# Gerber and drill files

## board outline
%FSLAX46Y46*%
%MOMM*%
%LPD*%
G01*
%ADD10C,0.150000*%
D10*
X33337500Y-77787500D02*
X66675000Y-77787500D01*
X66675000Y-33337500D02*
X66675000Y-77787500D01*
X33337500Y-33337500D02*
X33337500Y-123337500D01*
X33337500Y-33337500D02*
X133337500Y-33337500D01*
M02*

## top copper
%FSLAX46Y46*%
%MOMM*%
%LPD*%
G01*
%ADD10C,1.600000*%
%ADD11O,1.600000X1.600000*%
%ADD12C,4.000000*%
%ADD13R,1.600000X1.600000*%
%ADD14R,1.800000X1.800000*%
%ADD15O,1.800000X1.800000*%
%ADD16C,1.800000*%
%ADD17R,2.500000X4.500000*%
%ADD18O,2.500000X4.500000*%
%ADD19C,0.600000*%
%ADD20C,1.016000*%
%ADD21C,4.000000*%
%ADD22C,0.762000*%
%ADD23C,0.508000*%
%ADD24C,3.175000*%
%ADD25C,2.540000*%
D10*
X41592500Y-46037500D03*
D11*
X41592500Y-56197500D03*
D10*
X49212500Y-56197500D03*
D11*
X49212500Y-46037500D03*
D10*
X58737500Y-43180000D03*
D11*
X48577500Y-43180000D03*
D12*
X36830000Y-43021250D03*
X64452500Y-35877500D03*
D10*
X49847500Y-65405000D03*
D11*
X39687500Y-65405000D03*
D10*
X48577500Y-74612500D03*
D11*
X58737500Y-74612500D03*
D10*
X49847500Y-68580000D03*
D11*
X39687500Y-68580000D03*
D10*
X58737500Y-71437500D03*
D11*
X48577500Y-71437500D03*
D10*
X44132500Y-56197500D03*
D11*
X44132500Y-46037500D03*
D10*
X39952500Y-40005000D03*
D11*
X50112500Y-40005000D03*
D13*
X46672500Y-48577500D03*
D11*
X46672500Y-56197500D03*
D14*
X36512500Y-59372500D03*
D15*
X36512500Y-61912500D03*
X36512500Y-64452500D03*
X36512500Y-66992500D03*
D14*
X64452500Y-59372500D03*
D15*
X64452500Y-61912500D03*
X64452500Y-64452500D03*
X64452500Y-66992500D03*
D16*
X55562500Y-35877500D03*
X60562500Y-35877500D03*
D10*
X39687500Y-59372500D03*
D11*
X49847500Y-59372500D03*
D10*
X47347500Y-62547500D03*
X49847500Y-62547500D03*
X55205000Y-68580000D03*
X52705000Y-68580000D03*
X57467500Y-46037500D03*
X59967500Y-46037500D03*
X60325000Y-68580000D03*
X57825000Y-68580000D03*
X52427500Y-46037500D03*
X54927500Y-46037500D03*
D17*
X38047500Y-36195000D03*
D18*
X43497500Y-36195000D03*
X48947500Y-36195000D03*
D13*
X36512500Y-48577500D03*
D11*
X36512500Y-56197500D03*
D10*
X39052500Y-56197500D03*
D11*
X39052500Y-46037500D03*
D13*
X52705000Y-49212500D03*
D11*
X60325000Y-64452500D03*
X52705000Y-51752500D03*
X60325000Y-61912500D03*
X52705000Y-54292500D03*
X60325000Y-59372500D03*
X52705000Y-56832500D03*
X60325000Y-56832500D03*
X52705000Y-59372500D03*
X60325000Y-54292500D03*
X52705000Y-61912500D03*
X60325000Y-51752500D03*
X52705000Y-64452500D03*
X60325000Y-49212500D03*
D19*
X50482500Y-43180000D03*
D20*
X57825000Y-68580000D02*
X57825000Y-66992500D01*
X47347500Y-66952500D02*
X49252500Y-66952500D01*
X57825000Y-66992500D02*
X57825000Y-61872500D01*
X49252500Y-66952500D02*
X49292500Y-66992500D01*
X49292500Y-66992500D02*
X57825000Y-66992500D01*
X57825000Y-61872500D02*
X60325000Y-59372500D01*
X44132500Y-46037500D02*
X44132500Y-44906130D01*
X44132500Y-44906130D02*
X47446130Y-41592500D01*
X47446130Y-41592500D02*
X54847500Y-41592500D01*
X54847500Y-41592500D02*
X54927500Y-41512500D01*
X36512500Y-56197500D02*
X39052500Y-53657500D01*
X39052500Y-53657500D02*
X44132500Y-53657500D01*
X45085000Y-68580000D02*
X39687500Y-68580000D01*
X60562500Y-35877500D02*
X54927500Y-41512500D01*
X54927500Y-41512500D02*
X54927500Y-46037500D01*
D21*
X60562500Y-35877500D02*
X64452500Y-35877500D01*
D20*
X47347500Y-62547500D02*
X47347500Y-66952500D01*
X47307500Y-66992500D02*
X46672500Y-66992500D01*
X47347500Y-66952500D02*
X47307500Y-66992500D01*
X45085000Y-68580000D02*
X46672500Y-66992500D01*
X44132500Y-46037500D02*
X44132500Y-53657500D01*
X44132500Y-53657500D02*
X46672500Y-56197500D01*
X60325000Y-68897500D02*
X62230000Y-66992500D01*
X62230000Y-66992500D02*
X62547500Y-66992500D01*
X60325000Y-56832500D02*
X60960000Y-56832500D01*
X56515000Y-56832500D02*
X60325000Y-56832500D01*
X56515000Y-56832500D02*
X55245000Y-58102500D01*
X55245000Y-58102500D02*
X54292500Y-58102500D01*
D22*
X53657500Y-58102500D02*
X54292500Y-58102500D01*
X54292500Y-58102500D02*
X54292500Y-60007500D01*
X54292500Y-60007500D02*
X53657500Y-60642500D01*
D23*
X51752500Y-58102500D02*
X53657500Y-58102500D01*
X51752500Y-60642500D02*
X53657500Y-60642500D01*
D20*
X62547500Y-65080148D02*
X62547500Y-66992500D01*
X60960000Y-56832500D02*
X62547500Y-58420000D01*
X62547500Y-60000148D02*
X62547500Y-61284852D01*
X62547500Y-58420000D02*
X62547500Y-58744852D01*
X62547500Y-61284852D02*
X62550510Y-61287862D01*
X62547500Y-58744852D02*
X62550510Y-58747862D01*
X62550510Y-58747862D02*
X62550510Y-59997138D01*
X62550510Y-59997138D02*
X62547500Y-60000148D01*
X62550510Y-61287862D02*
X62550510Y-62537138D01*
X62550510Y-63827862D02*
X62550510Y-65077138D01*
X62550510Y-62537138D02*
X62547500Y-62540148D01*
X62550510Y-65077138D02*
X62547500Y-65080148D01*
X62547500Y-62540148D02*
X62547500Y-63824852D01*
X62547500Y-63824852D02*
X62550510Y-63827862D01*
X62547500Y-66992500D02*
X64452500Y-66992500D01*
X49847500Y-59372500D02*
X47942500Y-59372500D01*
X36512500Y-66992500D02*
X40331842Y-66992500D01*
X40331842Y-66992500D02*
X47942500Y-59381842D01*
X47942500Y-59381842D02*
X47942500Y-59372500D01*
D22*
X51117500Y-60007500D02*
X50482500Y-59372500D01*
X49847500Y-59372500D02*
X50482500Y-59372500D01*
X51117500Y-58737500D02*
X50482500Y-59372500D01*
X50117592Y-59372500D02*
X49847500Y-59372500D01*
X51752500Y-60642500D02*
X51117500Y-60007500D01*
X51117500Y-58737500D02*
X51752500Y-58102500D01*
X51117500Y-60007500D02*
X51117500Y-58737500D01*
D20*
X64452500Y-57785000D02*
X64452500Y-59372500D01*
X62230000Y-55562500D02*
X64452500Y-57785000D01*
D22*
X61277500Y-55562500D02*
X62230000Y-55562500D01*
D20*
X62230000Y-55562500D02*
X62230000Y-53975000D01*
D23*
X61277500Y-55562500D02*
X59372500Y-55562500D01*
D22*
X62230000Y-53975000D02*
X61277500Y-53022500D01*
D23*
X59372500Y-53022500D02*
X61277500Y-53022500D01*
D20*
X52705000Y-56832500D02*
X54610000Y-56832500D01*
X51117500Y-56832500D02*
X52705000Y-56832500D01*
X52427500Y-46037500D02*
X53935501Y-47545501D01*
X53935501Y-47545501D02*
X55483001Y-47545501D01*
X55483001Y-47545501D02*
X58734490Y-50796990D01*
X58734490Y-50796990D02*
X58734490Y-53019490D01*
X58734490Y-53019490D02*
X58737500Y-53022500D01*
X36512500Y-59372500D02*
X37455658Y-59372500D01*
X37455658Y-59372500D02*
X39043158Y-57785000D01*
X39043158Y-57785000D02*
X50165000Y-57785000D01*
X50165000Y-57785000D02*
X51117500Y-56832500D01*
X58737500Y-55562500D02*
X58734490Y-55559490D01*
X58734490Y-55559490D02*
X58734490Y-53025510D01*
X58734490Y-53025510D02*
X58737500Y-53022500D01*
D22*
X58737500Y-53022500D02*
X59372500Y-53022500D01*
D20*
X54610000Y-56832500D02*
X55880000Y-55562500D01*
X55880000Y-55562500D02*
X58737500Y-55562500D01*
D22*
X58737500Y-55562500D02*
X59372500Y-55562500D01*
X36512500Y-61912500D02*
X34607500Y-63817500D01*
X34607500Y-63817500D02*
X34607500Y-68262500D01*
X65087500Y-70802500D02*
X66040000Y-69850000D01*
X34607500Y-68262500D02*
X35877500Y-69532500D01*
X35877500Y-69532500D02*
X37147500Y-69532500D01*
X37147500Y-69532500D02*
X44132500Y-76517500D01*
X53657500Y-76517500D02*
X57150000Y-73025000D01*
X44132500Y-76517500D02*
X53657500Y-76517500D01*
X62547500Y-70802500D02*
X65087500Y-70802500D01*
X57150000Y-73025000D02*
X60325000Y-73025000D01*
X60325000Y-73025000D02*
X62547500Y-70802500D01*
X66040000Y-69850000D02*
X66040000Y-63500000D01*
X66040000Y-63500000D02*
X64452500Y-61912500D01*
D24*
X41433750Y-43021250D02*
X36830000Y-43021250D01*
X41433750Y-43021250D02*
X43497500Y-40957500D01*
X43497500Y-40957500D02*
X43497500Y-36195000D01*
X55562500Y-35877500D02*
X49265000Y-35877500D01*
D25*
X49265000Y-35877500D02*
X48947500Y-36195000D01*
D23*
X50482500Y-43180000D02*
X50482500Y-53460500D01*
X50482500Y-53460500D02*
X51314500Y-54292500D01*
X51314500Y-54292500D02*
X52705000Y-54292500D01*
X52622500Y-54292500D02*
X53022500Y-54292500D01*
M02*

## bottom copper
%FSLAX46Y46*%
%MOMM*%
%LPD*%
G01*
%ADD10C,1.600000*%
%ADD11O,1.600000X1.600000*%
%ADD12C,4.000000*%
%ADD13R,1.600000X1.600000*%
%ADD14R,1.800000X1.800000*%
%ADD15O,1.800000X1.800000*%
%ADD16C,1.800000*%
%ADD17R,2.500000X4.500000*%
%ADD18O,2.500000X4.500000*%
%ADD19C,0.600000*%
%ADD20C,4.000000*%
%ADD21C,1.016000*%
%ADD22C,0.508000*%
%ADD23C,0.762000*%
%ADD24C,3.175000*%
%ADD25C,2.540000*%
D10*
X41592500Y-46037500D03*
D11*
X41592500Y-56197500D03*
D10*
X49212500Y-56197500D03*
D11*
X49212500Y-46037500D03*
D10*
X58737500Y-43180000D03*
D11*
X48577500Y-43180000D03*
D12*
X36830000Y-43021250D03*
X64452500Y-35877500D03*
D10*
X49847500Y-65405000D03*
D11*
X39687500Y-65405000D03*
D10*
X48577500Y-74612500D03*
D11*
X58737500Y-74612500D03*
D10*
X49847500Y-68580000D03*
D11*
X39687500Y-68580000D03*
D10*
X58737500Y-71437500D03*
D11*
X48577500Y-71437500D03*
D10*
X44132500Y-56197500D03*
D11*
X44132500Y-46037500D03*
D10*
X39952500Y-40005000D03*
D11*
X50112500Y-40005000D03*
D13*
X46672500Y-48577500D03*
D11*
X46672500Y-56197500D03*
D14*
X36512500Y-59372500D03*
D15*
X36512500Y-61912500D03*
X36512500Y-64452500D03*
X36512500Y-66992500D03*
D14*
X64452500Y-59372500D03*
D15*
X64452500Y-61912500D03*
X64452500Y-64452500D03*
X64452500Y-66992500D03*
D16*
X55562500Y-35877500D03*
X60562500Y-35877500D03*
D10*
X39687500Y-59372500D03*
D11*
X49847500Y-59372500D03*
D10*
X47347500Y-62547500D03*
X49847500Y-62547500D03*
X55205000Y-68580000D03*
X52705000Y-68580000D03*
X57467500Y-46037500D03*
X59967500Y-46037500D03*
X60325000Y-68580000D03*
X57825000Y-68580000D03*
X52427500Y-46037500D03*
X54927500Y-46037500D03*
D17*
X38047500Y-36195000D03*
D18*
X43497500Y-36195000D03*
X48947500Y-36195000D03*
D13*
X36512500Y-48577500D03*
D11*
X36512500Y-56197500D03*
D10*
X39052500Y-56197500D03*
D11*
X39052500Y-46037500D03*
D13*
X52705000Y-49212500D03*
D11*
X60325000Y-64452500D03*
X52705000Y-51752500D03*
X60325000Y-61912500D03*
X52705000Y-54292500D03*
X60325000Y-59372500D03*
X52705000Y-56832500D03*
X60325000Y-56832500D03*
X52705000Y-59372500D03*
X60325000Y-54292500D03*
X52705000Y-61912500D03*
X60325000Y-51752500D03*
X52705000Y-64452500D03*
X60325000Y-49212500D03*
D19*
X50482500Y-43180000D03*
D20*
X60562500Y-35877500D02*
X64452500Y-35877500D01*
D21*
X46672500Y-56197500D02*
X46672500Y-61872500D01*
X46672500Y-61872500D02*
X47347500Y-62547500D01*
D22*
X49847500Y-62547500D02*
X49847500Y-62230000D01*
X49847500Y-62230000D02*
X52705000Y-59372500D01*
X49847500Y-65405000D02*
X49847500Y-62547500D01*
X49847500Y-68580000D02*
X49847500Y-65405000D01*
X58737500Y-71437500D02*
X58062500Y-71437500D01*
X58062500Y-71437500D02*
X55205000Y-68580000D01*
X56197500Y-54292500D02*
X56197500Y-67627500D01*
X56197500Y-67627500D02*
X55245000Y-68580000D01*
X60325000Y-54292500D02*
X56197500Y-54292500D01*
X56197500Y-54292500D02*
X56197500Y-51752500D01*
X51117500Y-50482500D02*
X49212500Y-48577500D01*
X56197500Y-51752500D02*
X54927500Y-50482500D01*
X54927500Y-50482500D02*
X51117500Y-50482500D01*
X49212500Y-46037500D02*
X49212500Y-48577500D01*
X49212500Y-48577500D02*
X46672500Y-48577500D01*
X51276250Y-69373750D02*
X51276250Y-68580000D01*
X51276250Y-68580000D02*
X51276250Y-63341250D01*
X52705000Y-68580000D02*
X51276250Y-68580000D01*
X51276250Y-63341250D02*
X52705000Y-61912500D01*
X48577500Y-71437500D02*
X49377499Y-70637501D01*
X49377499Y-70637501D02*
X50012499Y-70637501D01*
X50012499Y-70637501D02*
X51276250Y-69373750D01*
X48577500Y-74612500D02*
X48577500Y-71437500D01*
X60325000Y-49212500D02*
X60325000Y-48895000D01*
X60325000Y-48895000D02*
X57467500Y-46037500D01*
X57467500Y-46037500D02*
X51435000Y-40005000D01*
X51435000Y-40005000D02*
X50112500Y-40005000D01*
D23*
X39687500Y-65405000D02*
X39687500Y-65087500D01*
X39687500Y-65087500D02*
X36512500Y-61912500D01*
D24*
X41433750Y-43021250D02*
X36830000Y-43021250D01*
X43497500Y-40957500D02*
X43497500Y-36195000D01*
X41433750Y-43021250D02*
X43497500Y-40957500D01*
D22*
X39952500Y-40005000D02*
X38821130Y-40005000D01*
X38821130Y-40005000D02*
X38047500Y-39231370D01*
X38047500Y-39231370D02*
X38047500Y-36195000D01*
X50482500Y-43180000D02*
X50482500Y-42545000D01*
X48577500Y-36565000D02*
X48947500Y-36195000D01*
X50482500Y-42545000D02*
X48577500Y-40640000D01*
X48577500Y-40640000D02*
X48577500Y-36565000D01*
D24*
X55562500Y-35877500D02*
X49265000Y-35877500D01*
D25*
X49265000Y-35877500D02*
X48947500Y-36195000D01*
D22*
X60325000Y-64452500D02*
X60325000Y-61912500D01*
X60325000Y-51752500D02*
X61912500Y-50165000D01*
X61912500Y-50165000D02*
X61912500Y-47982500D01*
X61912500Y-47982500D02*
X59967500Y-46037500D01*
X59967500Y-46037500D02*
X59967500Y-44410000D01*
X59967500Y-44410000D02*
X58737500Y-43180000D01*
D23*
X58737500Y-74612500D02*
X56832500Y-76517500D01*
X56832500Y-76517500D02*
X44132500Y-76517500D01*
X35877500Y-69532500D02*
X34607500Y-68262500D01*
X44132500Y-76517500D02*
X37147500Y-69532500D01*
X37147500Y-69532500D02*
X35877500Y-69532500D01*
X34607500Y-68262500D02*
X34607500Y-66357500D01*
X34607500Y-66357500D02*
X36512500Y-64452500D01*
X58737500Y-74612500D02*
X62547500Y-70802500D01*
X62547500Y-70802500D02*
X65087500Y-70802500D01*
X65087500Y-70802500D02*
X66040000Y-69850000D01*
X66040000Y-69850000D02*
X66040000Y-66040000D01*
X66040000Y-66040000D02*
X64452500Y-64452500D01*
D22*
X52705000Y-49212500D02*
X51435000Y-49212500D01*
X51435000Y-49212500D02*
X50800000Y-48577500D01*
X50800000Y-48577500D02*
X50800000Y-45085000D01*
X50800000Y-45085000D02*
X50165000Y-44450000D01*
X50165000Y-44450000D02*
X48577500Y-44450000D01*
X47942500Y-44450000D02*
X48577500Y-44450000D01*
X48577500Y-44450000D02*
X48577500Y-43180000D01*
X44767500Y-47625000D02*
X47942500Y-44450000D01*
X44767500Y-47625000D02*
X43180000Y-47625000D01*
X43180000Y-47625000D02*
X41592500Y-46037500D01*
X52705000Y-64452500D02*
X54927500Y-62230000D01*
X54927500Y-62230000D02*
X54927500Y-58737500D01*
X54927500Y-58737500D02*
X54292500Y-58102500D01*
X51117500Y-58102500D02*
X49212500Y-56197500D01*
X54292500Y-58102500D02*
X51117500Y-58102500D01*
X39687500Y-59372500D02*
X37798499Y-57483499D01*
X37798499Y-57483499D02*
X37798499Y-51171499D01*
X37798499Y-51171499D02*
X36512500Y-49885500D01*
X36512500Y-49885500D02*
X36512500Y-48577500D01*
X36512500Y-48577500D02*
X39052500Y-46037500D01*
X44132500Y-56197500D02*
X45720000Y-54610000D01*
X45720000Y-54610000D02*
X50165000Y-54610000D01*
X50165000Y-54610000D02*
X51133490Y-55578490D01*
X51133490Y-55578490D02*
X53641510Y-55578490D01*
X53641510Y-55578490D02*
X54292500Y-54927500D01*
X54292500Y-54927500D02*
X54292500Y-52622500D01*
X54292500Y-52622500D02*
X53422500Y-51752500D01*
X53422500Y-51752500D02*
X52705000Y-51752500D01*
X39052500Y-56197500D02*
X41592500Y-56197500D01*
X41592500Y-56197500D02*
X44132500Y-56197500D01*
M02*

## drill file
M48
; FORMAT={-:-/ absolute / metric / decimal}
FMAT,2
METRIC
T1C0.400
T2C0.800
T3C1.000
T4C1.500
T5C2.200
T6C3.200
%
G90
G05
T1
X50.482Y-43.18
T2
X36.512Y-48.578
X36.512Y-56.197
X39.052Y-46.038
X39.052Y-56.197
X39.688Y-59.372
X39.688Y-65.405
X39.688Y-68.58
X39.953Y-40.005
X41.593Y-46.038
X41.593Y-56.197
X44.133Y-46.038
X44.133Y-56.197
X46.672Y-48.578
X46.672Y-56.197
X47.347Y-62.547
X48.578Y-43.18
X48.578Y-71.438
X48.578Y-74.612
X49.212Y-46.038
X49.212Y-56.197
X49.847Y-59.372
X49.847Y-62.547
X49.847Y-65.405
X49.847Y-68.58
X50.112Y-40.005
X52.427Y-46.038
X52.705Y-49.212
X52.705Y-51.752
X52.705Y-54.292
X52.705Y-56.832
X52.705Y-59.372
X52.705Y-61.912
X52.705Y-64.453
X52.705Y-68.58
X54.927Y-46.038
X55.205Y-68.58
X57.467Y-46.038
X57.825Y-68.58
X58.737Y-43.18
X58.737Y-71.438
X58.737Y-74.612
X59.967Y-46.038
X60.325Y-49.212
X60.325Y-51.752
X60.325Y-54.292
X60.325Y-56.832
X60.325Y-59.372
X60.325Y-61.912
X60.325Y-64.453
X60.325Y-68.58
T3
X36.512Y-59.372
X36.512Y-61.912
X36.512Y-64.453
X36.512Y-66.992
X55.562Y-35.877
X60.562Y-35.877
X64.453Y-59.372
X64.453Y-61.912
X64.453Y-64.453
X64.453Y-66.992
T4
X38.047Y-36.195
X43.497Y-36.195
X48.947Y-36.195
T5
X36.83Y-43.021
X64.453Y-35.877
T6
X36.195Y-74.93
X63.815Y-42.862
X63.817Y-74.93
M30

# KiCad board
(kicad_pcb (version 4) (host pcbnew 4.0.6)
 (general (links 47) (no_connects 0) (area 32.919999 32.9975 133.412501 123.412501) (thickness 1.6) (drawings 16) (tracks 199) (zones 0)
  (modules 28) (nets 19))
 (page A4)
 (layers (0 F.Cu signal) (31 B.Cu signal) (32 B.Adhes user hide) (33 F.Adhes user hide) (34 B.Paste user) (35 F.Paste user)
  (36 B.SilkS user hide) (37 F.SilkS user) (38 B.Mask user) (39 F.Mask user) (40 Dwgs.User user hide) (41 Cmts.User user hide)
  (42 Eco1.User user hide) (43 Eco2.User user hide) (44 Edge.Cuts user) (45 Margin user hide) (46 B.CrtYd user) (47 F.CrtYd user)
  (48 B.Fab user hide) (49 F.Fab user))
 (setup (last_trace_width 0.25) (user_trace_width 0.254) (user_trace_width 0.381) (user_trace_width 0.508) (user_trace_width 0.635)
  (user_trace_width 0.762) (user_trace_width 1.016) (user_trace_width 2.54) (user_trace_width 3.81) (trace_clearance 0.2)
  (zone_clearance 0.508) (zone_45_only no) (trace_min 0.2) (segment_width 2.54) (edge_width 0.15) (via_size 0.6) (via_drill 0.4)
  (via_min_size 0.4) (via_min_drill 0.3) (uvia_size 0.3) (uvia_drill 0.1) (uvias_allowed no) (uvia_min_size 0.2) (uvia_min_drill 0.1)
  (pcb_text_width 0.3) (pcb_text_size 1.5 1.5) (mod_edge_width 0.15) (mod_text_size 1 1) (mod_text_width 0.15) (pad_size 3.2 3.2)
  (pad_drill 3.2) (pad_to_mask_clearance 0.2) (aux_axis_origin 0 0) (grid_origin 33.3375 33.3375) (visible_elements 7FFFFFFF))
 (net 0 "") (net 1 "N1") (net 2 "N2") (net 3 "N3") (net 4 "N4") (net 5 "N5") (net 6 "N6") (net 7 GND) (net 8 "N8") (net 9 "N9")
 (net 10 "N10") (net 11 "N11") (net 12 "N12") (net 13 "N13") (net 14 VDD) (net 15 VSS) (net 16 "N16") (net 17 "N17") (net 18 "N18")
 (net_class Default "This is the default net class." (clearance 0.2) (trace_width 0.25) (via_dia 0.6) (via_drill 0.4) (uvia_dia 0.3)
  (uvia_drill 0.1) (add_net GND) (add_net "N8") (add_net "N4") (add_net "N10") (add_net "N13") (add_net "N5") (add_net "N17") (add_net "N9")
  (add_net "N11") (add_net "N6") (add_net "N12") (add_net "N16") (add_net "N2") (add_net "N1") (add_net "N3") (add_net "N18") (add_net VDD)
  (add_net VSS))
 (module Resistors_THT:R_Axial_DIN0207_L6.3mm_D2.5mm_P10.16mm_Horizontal (layer F.Cu) (at 41.5925 46.0375 270)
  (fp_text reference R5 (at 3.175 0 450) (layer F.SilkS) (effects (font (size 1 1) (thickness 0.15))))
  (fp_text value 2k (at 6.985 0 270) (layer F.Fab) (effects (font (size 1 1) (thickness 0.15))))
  (pad 1 thru_hole circle (at 0 0 270) (size 1.6 1.6) (drill 0.8) (layers *.Cu *.Mask) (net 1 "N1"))
  (pad 2 thru_hole oval (at 10.16 0 270) (size 1.6 1.6) (drill 0.8) (layers *.Cu *.Mask) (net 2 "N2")))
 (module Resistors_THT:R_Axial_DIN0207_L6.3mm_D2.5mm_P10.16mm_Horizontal (layer F.Cu) (at 49.2125 56.1975 90)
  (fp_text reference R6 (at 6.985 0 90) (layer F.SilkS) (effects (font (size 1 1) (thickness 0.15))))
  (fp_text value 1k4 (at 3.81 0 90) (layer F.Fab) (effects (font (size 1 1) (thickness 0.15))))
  (pad 1 thru_hole circle (at 0 0 90) (size 1.6 1.6) (drill 0.8) (layers *.Cu *.Mask) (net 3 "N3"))
  (pad 2 thru_hole oval (at 10.16 0 90) (size 1.6 1.6) (drill 0.8) (layers *.Cu *.Mask) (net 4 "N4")))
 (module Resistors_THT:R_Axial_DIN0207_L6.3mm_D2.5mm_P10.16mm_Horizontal (layer F.Cu) (at 58.7375 43.18 180)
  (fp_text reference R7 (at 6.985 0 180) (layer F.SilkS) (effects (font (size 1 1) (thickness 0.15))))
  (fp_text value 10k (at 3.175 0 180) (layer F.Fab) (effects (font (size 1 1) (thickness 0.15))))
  (pad 1 thru_hole circle (at 0 0 180) (size 1.6 1.6) (drill 0.8) (layers *.Cu *.Mask) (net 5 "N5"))
  (pad 2 thru_hole oval (at 10.16 0 180) (size 1.6 1.6) (drill 0.8) (layers *.Cu *.Mask) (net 1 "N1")))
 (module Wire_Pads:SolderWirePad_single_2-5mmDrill (layer F.Cu) (at 36.83 43.02125)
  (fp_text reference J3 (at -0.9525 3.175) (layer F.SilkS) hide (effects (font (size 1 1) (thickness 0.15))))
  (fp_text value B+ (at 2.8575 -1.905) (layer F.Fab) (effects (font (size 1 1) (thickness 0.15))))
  (pad 1 thru_hole circle (at 0 0) (size 4 4) (drill 2.2) (layers *.Cu *.Mask) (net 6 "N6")))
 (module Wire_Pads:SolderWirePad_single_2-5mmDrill (layer F.Cu) (at 64.4525 35.8775)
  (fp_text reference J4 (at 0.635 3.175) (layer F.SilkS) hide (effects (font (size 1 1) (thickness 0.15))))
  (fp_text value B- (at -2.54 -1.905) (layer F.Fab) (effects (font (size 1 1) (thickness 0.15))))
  (pad 1 thru_hole circle (at 0 0) (size 4 4) (drill 2.2) (layers *.Cu *.Mask) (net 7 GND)))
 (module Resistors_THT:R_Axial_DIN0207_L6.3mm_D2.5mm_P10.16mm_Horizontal (layer F.Cu) (at 49.8475 65.405 180)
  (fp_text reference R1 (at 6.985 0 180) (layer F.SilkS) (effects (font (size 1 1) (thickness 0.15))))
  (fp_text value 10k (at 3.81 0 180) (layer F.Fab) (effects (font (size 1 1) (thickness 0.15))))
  (pad 1 thru_hole circle (at 0 0 180) (size 1.6 1.6) (drill 0.8) (layers *.Cu *.Mask) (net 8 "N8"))
  (pad 2 thru_hole oval (at 10.16 0 180) (size 1.6 1.6) (drill 0.8) (layers *.Cu *.Mask) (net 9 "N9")))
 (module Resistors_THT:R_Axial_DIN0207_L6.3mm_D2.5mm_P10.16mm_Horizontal (layer F.Cu) (at 48.5775 74.6125)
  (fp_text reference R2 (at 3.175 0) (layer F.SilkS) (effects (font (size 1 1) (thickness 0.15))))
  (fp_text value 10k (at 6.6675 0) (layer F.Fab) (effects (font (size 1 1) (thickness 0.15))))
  (pad 1 thru_hole circle (at 0 0) (size 1.6 1.6) (drill 0.8) (layers *.Cu *.Mask) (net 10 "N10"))
  (pad 2 thru_hole oval (at 10.16 0) (size 1.6 1.6) (drill 0.8) (layers *.Cu *.Mask) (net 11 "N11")))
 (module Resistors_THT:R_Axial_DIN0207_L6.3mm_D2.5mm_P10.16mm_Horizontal (layer F.Cu) (at 49.8475 68.58 180)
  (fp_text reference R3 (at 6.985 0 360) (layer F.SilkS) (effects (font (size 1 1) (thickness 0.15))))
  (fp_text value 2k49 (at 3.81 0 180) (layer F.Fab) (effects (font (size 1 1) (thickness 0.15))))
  (pad 1 thru_hole circle (at 0 0 180) (size 1.6 1.6) (drill 0.8) (layers *.Cu *.Mask) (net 8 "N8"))
  (pad 2 thru_hole oval (at 10.16 0 180) (size 1.6 1.6) (drill 0.8) (layers *.Cu *.Mask) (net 7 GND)))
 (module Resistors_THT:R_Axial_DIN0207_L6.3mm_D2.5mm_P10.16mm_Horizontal (layer F.Cu) (at 58.7375 71.4375 180)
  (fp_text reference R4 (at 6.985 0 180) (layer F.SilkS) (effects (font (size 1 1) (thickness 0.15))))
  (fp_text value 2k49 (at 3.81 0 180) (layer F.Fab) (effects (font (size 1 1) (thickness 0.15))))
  (pad 1 thru_hole circle (at 0 0 180) (size 1.6 1.6) (drill 0.8) (layers *.Cu *.Mask) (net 4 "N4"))
  (pad 2 thru_hole oval (at 10.16 0 180) (size 1.6 1.6) (drill 0.8) (layers *.Cu *.Mask) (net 10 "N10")))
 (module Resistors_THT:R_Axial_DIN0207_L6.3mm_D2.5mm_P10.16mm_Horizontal (layer F.Cu) (at 44.1325 56.1975 90)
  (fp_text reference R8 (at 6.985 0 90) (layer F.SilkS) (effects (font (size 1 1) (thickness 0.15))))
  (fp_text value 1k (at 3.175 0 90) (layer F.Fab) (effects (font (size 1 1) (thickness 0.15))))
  (pad 1 thru_hole circle (at 0 0 90) (size 1.6 1.6) (drill 0.8) (layers *.Cu *.Mask) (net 2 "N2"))
  (pad 2 thru_hole oval (at 10.16 0 90) (size 1.6 1.6) (drill 0.8) (layers *.Cu *.Mask) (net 7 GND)))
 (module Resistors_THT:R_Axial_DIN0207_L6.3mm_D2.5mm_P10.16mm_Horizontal (layer F.Cu) (at 39.9525 40.005)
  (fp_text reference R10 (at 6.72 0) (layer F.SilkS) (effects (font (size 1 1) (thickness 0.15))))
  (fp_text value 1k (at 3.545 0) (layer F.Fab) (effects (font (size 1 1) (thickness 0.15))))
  (pad 1 thru_hole circle (at 0 0) (size 1.6 1.6) (drill 0.8) (layers *.Cu *.Mask) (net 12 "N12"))
  (pad 2 thru_hole oval (at 10.16 0) (size 1.6 1.6) (drill 0.8) (layers *.Cu *.Mask) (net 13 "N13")))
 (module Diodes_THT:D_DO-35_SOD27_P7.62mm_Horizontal (layer F.Cu) (at 46.6725 48.5775 270)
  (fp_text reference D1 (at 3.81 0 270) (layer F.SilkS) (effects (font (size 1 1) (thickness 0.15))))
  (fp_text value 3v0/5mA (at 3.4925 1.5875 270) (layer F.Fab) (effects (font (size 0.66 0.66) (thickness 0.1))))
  (pad 1 thru_hole rect (at 0 0 270) (size 1.6 1.6) (drill 0.8) (layers *.Cu *.Mask) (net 4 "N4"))
  (pad 2 thru_hole oval (at 7.62 0 270) (size 1.6 1.6) (drill 0.8) (layers *.Cu *.Mask) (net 7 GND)))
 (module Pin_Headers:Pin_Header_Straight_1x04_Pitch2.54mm (layer F.Cu) (at 36.5125 59.3725)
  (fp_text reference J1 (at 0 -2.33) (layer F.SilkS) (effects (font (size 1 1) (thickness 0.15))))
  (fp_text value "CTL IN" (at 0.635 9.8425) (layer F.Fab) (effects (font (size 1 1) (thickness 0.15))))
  (pad 1 thru_hole rect (at 0 0) (size 1.8 1.8) (drill 1) (layers *.Cu *.Mask) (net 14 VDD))
  (pad 2 thru_hole oval (at 0 2.54) (size 1.8 1.8) (drill 1) (layers *.Cu *.Mask) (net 9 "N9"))
  (pad 3 thru_hole oval (at 0 5.08) (size 1.8 1.8) (drill 1) (layers *.Cu *.Mask) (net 11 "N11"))
  (pad 4 thru_hole oval (at 0 7.62) (size 1.8 1.8) (drill 1) (layers *.Cu *.Mask) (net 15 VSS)))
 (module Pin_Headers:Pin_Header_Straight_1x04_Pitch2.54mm (layer F.Cu) (at 64.4525 59.3725)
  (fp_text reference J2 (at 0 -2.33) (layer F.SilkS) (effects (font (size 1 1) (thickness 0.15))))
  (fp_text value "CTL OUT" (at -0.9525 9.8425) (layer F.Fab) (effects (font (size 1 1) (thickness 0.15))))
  (pad 1 thru_hole rect (at 0 0) (size 1.8 1.8) (drill 1) (layers *.Cu *.Mask) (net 14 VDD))
  (pad 2 thru_hole oval (at 0 2.54) (size 1.8 1.8) (drill 1) (layers *.Cu *.Mask) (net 9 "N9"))
  (pad 3 thru_hole oval (at 0 5.08) (size 1.8 1.8) (drill 1) (layers *.Cu *.Mask) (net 11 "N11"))
  (pad 4 thru_hole oval (at 0 7.62) (size 1.8 1.8) (drill 1) (layers *.Cu *.Mask) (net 15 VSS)))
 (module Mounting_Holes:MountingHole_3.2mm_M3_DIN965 (layer F.Cu) (at 63.81496 42.8625)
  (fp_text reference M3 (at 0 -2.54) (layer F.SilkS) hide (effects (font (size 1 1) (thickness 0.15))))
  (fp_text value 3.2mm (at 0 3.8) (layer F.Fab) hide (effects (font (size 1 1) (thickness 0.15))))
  (pad "" np_thru_hole circle (at 0 0) (size 3.2 3.2) (drill 3.2) (layers *.Cu *.Mask)))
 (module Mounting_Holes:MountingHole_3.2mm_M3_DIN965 (layer F.Cu) (at 36.195 74.93)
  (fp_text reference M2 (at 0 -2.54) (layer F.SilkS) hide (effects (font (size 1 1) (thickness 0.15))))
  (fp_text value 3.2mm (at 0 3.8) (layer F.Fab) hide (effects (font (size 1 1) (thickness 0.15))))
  (pad 1 np_thru_hole circle (at 0 0) (size 3.2 3.2) (drill 3.2) (layers *.Cu *.Mask)))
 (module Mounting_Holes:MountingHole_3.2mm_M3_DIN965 (layer F.Cu) (at 63.8175 74.93)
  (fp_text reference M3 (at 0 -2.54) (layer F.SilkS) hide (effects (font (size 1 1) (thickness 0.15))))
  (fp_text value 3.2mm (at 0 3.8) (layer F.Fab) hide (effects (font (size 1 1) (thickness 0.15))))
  (pad 1 np_thru_hole circle (at 0 0) (size 3.2 3.2) (drill 3.2) (layers *.Cu *.Mask)))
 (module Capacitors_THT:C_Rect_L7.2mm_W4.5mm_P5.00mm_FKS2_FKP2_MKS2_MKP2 (layer F.Cu) (at 55.5625 35.8775)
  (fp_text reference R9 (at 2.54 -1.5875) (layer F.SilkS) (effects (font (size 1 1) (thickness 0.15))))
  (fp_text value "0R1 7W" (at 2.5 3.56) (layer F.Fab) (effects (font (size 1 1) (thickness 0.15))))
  (pad 1 thru_hole circle (at 0 0) (size 1.8 1.8) (drill 1) (layers *.Cu *.Mask) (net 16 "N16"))
  (pad 2 thru_hole circle (at 5 0) (size 1.8 1.8) (drill 1) (layers *.Cu *.Mask) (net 7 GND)))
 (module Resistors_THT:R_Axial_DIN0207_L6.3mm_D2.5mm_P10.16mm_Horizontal (layer F.Cu) (at 39.6875 59.3725)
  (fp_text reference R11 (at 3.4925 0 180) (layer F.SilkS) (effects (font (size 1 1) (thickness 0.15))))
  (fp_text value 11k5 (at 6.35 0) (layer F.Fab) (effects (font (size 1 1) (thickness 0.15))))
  (pad 1 thru_hole circle (at 0 0) (size 1.6 1.6) (drill 0.8) (layers *.Cu *.Mask) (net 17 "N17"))
  (pad 2 thru_hole oval (at 10.16 0) (size 1.6 1.6) (drill 0.8) (layers *.Cu *.Mask) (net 15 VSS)))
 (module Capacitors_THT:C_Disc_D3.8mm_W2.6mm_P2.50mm (layer F.Cu) (at 47.3475 62.5475)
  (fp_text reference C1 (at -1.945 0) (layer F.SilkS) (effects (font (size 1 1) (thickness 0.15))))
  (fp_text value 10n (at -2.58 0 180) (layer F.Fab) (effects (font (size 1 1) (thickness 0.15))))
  (pad 1 thru_hole circle (at 0 0) (size 1.6 1.6) (drill 0.8) (layers *.Cu *.Mask) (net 7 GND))
  (pad 2 thru_hole circle (at 2.5 0) (size 1.6 1.6) (drill 0.8) (layers *.Cu *.Mask) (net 8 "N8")))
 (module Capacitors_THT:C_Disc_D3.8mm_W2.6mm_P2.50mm (layer F.Cu) (at 55.205 68.58 180)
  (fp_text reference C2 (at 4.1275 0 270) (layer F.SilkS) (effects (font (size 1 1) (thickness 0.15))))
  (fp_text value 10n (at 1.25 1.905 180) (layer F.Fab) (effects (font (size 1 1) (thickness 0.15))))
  (pad 1 thru_hole circle (at 0 0 180) (size 1.6 1.6) (drill 0.8) (layers *.Cu *.Mask) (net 4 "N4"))
  (pad 2 thru_hole circle (at 2.5 0 180) (size 1.6 1.6) (drill 0.8) (layers *.Cu *.Mask) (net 10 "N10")))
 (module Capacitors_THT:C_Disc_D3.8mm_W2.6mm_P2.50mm (layer F.Cu) (at 57.4675 46.0375)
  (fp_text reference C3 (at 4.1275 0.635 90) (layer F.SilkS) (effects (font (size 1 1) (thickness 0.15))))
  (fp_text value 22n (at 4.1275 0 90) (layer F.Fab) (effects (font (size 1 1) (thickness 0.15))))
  (pad 1 thru_hole circle (at 0 0) (size 1.6 1.6) (drill 0.8) (layers *.Cu *.Mask) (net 13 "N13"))
  (pad 2 thru_hole circle (at 2.5 0) (size 1.6 1.6) (drill 0.8) (layers *.Cu *.Mask) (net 5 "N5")))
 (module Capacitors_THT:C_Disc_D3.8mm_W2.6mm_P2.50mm (layer F.Cu) (at 60.325 68.58 180)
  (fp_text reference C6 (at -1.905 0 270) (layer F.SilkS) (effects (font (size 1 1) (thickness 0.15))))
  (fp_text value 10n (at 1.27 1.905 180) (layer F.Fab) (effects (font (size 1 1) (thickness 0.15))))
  (pad 1 thru_hole circle (at 0 0 180) (size 1.6 1.6) (drill 0.8) (layers *.Cu *.Mask) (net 15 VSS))
  (pad 2 thru_hole circle (at 2.5 0 180) (size 1.6 1.6) (drill 0.8) (layers *.Cu *.Mask) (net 7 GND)))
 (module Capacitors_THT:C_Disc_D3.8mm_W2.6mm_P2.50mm (layer F.Cu) (at 52.4275 46.0375)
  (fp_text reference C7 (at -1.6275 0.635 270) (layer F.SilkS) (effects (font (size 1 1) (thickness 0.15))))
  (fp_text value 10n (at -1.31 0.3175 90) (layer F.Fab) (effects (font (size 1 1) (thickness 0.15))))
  (pad 1 thru_hole circle (at 0 0) (size 1.6 1.6) (drill 0.8) (layers *.Cu *.Mask) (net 14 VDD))
  (pad 2 thru_hole circle (at 2.5 0) (size 1.6 1.6) (drill 0.8) (layers *.Cu *.Mask) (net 7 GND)))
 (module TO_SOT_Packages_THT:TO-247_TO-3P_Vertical (layer F.Cu) (at 38.0475 36.195)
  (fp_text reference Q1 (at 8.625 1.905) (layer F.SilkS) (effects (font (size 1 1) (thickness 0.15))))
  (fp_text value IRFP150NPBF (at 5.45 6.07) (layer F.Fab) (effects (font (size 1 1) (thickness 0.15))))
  (pad 1 thru_hole rect (at 0 0) (size 2.5 4.5) (drill 1.5) (layers *.Cu *.Mask) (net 12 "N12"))
  (pad 2 thru_hole oval (at 5.45 0) (size 2.5 4.5) (drill 1.5) (layers *.Cu *.Mask) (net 6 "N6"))
  (pad 3 thru_hole oval (at 10.9 0) (size 2.5 4.5) (drill 1.5) (layers *.Cu *.Mask) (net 16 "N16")))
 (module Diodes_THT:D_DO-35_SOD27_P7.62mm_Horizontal (layer F.Cu) (at 36.5125 48.5775 270)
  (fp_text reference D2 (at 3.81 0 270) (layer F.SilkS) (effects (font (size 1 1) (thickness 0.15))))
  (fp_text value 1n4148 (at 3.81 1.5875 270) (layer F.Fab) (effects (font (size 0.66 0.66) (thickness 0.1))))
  (pad 1 thru_hole rect (at 0 0 270) (size 1.6 1.6) (drill 0.8) (layers *.Cu *.Mask) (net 17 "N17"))
  (pad 2 thru_hole oval (at 7.62 0 270) (size 1.6 1.6) (drill 0.8) (layers *.Cu *.Mask) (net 7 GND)))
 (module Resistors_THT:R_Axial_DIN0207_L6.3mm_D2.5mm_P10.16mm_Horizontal (layer F.Cu) (at 39.0525 56.1975 90)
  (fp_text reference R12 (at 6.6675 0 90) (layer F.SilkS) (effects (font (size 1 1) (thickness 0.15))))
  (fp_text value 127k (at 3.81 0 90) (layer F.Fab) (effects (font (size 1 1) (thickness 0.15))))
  (pad 1 thru_hole circle (at 0 0 90) (size 1.6 1.6) (drill 0.8) (layers *.Cu *.Mask) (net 2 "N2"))
  (pad 2 thru_hole oval (at 10.16 0 90) (size 1.6 1.6) (drill 0.8) (layers *.Cu *.Mask) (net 17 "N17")))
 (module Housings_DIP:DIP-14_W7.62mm (layer F.Cu) (at 52.705 49.2125)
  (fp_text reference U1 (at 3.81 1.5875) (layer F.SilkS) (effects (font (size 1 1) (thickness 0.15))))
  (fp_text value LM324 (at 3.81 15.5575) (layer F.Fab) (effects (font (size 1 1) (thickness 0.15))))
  (pad 1 thru_hole rect (at 0 0) (size 1.6 1.6) (drill 0.8) (layers *.Cu *.Mask) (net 1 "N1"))
  (pad 8 thru_hole oval (at 7.62 15.24) (size 1.6 1.6) (drill 0.8) (layers *.Cu *.Mask) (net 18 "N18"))
  (pad 2 thru_hole oval (at 0 2.54) (size 1.6 1.6) (drill 0.8) (layers *.Cu *.Mask) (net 2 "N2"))
  (pad 9 thru_hole oval (at 7.62 12.7) (size 1.6 1.6) (drill 0.8) (layers *.Cu *.Mask) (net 18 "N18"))
  (pad 3 thru_hole oval (at 0 5.08) (size 1.6 1.6) (drill 0.8) (layers *.Cu *.Mask) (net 16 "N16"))
  (pad 10 thru_hole oval (at 7.62 10.16) (size 1.6 1.6) (drill 0.8) (layers *.Cu *.Mask) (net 7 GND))
  (pad 4 thru_hole oval (at 0 7.62) (size 1.6 1.6) (drill 0.8) (layers *.Cu *.Mask) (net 14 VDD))
  (pad 11 thru_hole oval (at 7.62 7.62) (size 1.6 1.6) (drill 0.8) (layers *.Cu *.Mask) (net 15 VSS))
  (pad 5 thru_hole oval (at 0 10.16) (size 1.6 1.6) (drill 0.8) (layers *.Cu *.Mask) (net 8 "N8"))
  (pad 12 thru_hole oval (at 7.62 5.08) (size 1.6 1.6) (drill 0.8) (layers *.Cu *.Mask) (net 4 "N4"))
  (pad 6 thru_hole oval (at 0 12.7) (size 1.6 1.6) (drill 0.8) (layers *.Cu *.Mask) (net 10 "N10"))
  (pad 13 thru_hole oval (at 7.62 2.54) (size 1.6 1.6) (drill 0.8) (layers *.Cu *.Mask) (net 5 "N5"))
  (pad 7 thru_hole oval (at 0 15.24) (size 1.6 1.6) (drill 0.8) (layers *.Cu *.Mask) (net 3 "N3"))
  (pad 14 thru_hole oval (at 7.62 0) (size 1.6 1.6) (drill 0.8) (layers *.Cu *.Mask) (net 13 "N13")))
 (gr_line (start 33.3375 77.7875) (end 66.675 77.7875) (layer Edge.Cuts) (width 0.15))
 (gr_line (start 66.675 33.3375) (end 66.675 77.7875) (layer Edge.Cuts) (width 0.15))
 (gr_line (start 33.3375 33.3375) (end 33.3375 123.3375) (layer Edge.Cuts) (width 0.15))
 (gr_line (start 33.3375 33.3375) (end 133.3375 33.3375) (layer Edge.Cuts) (width 0.15))
 (segment (start 57.825 68.58) (end 57.825 66.9925) (width 1.016) (layer F.Cu) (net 7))
 (segment (start 47.3475 66.9525) (end 49.2525 66.9525) (width 1.016) (layer F.Cu) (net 7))
 (segment (start 57.825 66.9925) (end 57.825 61.8725) (width 1.016) (layer F.Cu) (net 7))
 (segment (start 49.2525 66.9525) (end 49.2925 66.9925) (width 1.016) (layer F.Cu) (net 7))
 (segment (start 49.2925 66.9925) (end 57.825 66.9925) (width 1.016) (layer F.Cu) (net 7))
 (segment (start 57.825 61.8725) (end 60.325 59.3725) (width 1.016) (layer F.Cu) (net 7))
 (segment (start 44.1325 46.0375) (end 44.1325 44.90613) (width 1.016) (layer F.Cu) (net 7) (status 10))
 (segment (start 44.1325 44.90613) (end 47.44613 41.5925) (width 1.016) (layer F.Cu) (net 7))
 (segment (start 47.44613 41.5925) (end 54.8475 41.5925) (width 1.016) (layer F.Cu) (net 7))
 (segment (start 54.8475 41.5925) (end 54.9275 41.5125) (width 1.016) (layer F.Cu) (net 7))
 (segment (start 36.5125 56.1975) (end 39.0525 53.6575) (width 1.016) (layer F.Cu) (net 7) (status 10))
 (segment (start 39.0525 53.6575) (end 44.1325 53.6575) (width 1.016) (layer F.Cu) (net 7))
 (segment (start 45.085 68.58) (end 39.6875 68.58) (width 1.016) (layer F.Cu) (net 7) (status 20))
 (segment (start 60.5625 35.8775) (end 54.9275 41.5125) (width 1.016) (layer F.Cu) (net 7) (status 10))
 (segment (start 54.9275 41.5125) (end 54.9275 46.0375) (width 1.016) (layer F.Cu) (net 7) (status 20))
 (segment (start 60.5625 35.8775) (end 64.4525 35.8775) (width 4) (layer B.Cu) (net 7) (status 30))
 (segment (start 60.5625 35.8775) (end 64.4525 35.8775) (width 4) (layer F.Cu) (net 7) (status 30))
 (segment (start 46.6725 56.1975) (end 46.6725 61.8725) (width 1.016) (layer B.Cu) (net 7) (status 10))
 (segment (start 46.6725 61.8725) (end 47.3475 62.5475) (width 1.016) (layer B.Cu) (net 7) (status 20))
 (segment (start 47.3475 62.5475) (end 47.3475 66.9525) (width 1.016) (layer F.Cu) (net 7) (status 10))
 (segment (start 47.3075 66.9925) (end 46.6725 66.9925) (width 1.016) (layer F.Cu) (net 7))
 (segment (start 47.3475 66.9525) (end 47.3075 66.9925) (width 1.016) (layer F.Cu) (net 7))
 (segment (start 45.085 68.58) (end 46.6725 66.9925) (width 1.016) (layer F.Cu) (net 7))
 (segment (start 44.1325 46.0375) (end 44.1325 53.6575) (width 1.016) (layer F.Cu) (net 7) (status 10))
 (segment (start 44.1325 53.6575) (end 46.6725 56.1975) (width 1.016) (layer F.Cu) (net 7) (status 20))
 (segment (start 49.8475 62.5475) (end 49.8475 62.23) (width 0.508) (layer B.Cu) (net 8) (status 30))
 (segment (start 49.8475 62.23) (end 52.705 59.3725) (width 0.508) (layer B.Cu) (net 8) (status 30))
 (segment (start 49.8475 65.405) (end 49.8475 62.5475) (width 0.508) (layer B.Cu) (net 8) (status 30))
 (segment (start 49.8475 68.58) (end 49.8475 65.405) (width 0.508) (layer B.Cu) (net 8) (status 30))
 (segment (start 58.7375 71.4375) (end 58.0625 71.4375) (width 0.508) (layer B.Cu) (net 4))
 (segment (start 58.0625 71.4375) (end 55.205 68.58) (width 0.508) (layer B.Cu) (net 4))
 (segment (start 56.1975 54.2925) (end 56.1975 67.6275) (width 0.508) (layer B.Cu) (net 4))
 (segment (start 56.1975 67.6275) (end 55.245 68.58) (width 0.508) (layer B.Cu) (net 4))
 (segment (start 60.325 54.2925) (end 56.1975 54.2925) (width 0.508) (layer B.Cu) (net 4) (status 10))
 (segment (start 56.1975 54.2925) (end 56.1975 51.7525) (width 0.508) (layer B.Cu) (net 4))
 (segment (start 51.1175 50.4825) (end 49.2125 48.5775) (width 0.508) (layer B.Cu) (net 4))
 (segment (start 56.1975 51.7525) (end 54.9275 50.4825) (width 0.508) (layer B.Cu) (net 4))
 (segment (start 54.9275 50.4825) (end 51.1175 50.4825) (width 0.508) (layer B.Cu) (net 4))
 (segment (start 49.2125 46.0375) (end 49.2125 48.5775) (width 0.508) (layer B.Cu) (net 4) (status 10))
 (segment (start 49.2125 48.5775) (end 46.6725 48.5775) (width 0.508) (layer B.Cu) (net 4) (status 20))
 (segment (start 51.27625 69.37375) (end 51.27625 68.58) (width 0.508) (layer B.Cu) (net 10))
 (segment (start 51.27625 68.58) (end 51.27625 63.34125) (width 0.508) (layer B.Cu) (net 10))
 (segment (start 52.705 68.58) (end 51.27625 68.58) (width 0.508) (layer B.Cu) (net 10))
 (segment (start 51.27625 63.34125) (end 52.705 61.9125) (width 0.508) (layer B.Cu) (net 10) (status 20))
 (segment (start 48.5775 71.4375) (end 49.377499 70.637501) (width 0.508) (layer B.Cu) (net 10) (status 10))
 (segment (start 49.377499 70.637501) (end 50.012499 70.637501) (width 0.508) (layer B.Cu) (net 10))
 (segment (start 50.012499 70.637501) (end 51.27625 69.37375) (width 0.508) (layer B.Cu) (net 10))
 (segment (start 48.5775 74.6125) (end 48.5775 71.4375) (width 0.508) (layer B.Cu) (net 10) (status 30))
 (segment (start 60.325 49.2125) (end 60.325 48.895) (width 0.508) (layer B.Cu) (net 13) (status 30))
 (segment (start 60.325 48.895) (end 57.4675 46.0375) (width 0.508) (layer B.Cu) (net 13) (status 30))
 (segment (start 57.4675 46.0375) (end 51.435 40.005) (width 0.508) (layer B.Cu) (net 13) (status 10))
 (segment (start 51.435 40.005) (end 50.1125 40.005) (width 0.508) (layer B.Cu) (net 13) (status 20))
 (segment (start 60.325 68.8975) (end 62.23 66.9925) (width 1.016) (layer F.Cu) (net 15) (status 10))
 (segment (start 62.23 66.9925) (end 62.5475 66.9925) (width 1.016) (layer F.Cu) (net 15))
 (segment (start 60.325 56.8325) (end 60.96 56.8325) (width 1.016) (layer F.Cu) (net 15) (status 30))
 (segment (start 56.515 56.8325) (end 60.325 56.8325) (width 1.016) (layer F.Cu) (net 15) (status 20))
 (segment (start 56.515 56.8325) (end 55.245 58.1025) (width 1.016) (layer F.Cu) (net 15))
 (segment (start 55.245 58.1025) (end 54.2925 58.1025) (width 1.016) (layer F.Cu) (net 15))
 (segment (start 53.6575 58.1025) (end 54.2925 58.1025) (width 0.762) (layer F.Cu) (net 15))
 (segment (start 54.2925 58.1025) (end 54.2925 60.0075) (width 0.762) (layer F.Cu) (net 15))
 (segment (start 54.2925 60.0075) (end 53.6575 60.6425) (width 0.762) (layer F.Cu) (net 15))
 (segment (start 51.7525 58.1025) (end 53.6575 58.1025) (width 0.508) (layer F.Cu) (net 15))
 (segment (start 51.7525 60.6425) (end 53.6575 60.6425) (width 0.508) (layer F.Cu) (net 15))
 (segment (start 62.5475 65.080148) (end 62.5475 66.9925) (width 1.016) (layer F.Cu) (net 15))
 (segment (start 60.96 56.8325) (end 62.5475 58.42) (width 1.016) (layer F.Cu) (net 15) (status 10))
 (segment (start 62.5475 60.000148) (end 62.5475 61.284852) (width 1.016) (layer F.Cu) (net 15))
 (segment (start 62.5475 58.42) (end 62.5475 58.744852) (width 1.016) (layer F.Cu) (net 15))
 (segment (start 62.5475 61.284852) (end 62.55051 61.287862) (width 1.016) (layer F.Cu) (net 15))
 (segment (start 62.5475 58.744852) (end 62.55051 58.747862) (width 1.016) (layer F.Cu) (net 15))
 (segment (start 62.55051 58.747862) (end 62.55051 59.997138) (width 1.016) (layer F.Cu) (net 15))
 (segment (start 62.55051 59.997138) (end 62.5475 60.000148) (width 1.016) (layer F.Cu) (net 15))
 (segment (start 62.55051 61.287862) (end 62.55051 62.537138) (width 1.016) (layer F.Cu) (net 15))
 (segment (start 62.55051 63.827862) (end 62.55051 65.077138) (width 1.016) (layer F.Cu) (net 15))
 (segment (start 62.55051 62.537138) (end 62.5475 62.540148) (width 1.016) (layer F.Cu) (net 15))
 (segment (start 62.55051 65.077138) (end 62.5475 65.080148) (width 1.016) (layer F.Cu) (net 15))
 (segment (start 62.5475 62.540148) (end 62.5475 63.824852) (width 1.016) (layer F.Cu) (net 15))
 (segment (start 62.5475 63.824852) (end 62.55051 63.827862) (width 1.016) (layer F.Cu) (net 15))
 (segment (start 62.5475 66.9925) (end 64.4525 66.9925) (width 1.016) (layer F.Cu) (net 15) (status 20))
 (segment (start 49.8475 59.3725) (end 47.9425 59.3725) (width 1.016) (layer F.Cu) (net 15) (status 10))
 (segment (start 36.5125 66.9925) (end 40.331842 66.9925) (width 1.016) (layer F.Cu) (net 15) (status 10))
 (segment (start 40.331842 66.9925) (end 47.9425 59.381842) (width 1.016) (layer F.Cu) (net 15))
 (segment (start 47.9425 59.381842) (end 47.9425 59.3725) (width 1.016) (layer F.Cu) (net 15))
 (segment (start 51.1175 60.0075) (end 50.4825 59.3725) (width 0.762) (layer F.Cu) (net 15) (status 20))
 (segment (start 49.8475 59.3725) (end 50.4825 59.3725) (width 0.762) (layer F.Cu) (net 15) (status 30))
 (segment (start 51.1175 58.7375) (end 50.4825 59.3725) (width 0.762) (layer F.Cu) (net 15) (status 20))
 (segment (start 50.117592 59.3725) (end 49.8475 59.3725) (width 0.762) (layer F.Cu) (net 15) (status 30))
 (segment (start 51.7525 60.6425) (end 51.1175 60.0075) (width 0.762) (layer F.Cu) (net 15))
 (segment (start 51.1175 58.7375) (end 51.7525 58.1025) (width 0.762) (layer F.Cu) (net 15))
 (segment (start 51.1175 60.0075) (end 51.1175 58.7375) (width 0.762) (layer F.Cu) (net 15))
 (segment (start 64.4525 57.785) (end 64.4525 59.3725) (width 1.016) (layer F.Cu) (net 14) (status 20))
 (segment (start 62.23 55.5625) (end 64.4525 57.785) (width 1.016) (layer F.Cu) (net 14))
 (segment (start 61.2775 55.5625) (end 62.23 55.5625) (width 0.762) (layer F.Cu) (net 14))
 (segment (start 62.23 55.5625) (end 62.23 53.975) (width 1.016) (layer F.Cu) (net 14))
 (segment (start 61.2775 55.5625) (end 59.3725 55.5625) (width 0.508) (layer F.Cu) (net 14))
 (segment (start 62.23 53.975) (end 61.2775 53.0225) (width 0.762) (layer F.Cu) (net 14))
 (segment (start 59.3725 53.0225) (end 61.2775 53.0225) (width 0.508) (layer F.Cu) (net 14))
 (segment (start 52.705 56.8325) (end 54.61 56.8325) (width 1.016) (layer F.Cu) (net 14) (status 10))
 (segment (start 51.1175 56.8325) (end 52.705 56.8325) (width 1.016) (layer F.Cu) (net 14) (status 20))
 (segment (start 52.4275 46.0375) (end 53.935501 47.545501) (width 1.016) (layer F.Cu) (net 14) (status 10))
 (segment (start 53.935501 47.545501) (end 55.483001 47.545501) (width 1.016) (layer F.Cu) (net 14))
 (segment (start 55.483001 47.545501) (end 58.73449 50.79699) (width 1.016) (layer F.Cu) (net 14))
 (segment (start 58.73449 50.79699) (end 58.73449 53.01949) (width 1.016) (layer F.Cu) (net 14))
 (segment (start 58.73449 53.01949) (end 58.7375 53.0225) (width 1.016) (layer F.Cu) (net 14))
 (segment (start 36.5125 59.3725) (end 37.455658 59.3725) (width 1.016) (layer F.Cu) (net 14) (status 10))
 (segment (start 37.455658 59.3725) (end 39.043158 57.785) (width 1.016) (layer F.Cu) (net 14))
 (segment (start 39.043158 57.785) (end 50.165 57.785) (width 1.016) (layer F.Cu) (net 14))
 (segment (start 50.165 57.785) (end 51.1175 56.8325) (width 1.016) (layer F.Cu) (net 14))
 (segment (start 58.7375 55.5625) (end 58.73449 55.55949) (width 1.016) (layer F.Cu) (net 14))
 (segment (start 58.73449 55.55949) (end 58.73449 53.02551) (width 1.016) (layer F.Cu) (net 14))
 (segment (start 58.73449 53.02551) (end 58.7375 53.0225) (width 1.016) (layer F.Cu) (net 14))
 (segment (start 58.7375 53.0225) (end 59.3725 53.0225) (width 0.762) (layer F.Cu) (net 14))
 (segment (start 54.61 56.8325) (end 55.88 55.5625) (width 1.016) (layer F.Cu) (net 14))
 (segment (start 55.88 55.5625) (end 58.7375 55.5625) (width 1.016) (layer F.Cu) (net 14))
 (segment (start 58.7375 55.5625) (end 59.3725 55.5625) (width 0.762) (layer F.Cu) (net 14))
 (segment (start 36.5125 61.9125) (end 34.6075 63.8175) (width 0.762) (layer F.Cu) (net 9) (status 10))
 (segment (start 34.6075 63.8175) (end 34.6075 68.2625) (width 0.762) (layer F.Cu) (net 9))
 (segment (start 65.0875 70.8025) (end 66.04 69.85) (width 0.762) (layer F.Cu) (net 9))
 (segment (start 34.6075 68.2625) (end 35.8775 69.5325) (width 0.762) (layer F.Cu) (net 9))
 (segment (start 35.8775 69.5325) (end 37.1475 69.5325) (width 0.762) (layer F.Cu) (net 9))
 (segment (start 37.1475 69.5325) (end 44.1325 76.5175) (width 0.762) (layer F.Cu) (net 9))
 (segment (start 53.6575 76.5175) (end 57.15 73.025) (width 0.762) (layer F.Cu) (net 9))
 (segment (start 44.1325 76.5175) (end 53.6575 76.5175) (width 0.762) (layer F.Cu) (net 9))
 (segment (start 62.5475 70.8025) (end 65.0875 70.8025) (width 0.762) (layer F.Cu) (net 9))
 (segment (start 57.15 73.025) (end 60.325 73.025) (width 0.762) (layer F.Cu) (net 9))
 (segment (start 60.325 73.025) (end 62.5475 70.8025) (width 0.762) (layer F.Cu) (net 9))
 (segment (start 66.04 69.85) (end 66.04 63.5) (width 0.762) (layer F.Cu) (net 9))
 (segment (start 66.04 63.5) (end 64.4525 61.9125) (width 0.762) (layer F.Cu) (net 9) (status 20))
 (segment (start 39.6875 65.405) (end 39.6875 65.0875) (width 0.762) (layer B.Cu) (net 9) (status 30))
 (segment (start 39.6875 65.0875) (end 36.5125 61.9125) (width 0.762) (layer B.Cu) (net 9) (status 30))
 (segment (start 41.43375 43.02125) (end 36.83 43.02125) (width 3.175) (layer B.Cu) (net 6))
 (segment (start 41.43375 43.02125) (end 36.83 43.02125) (width 3.175) (layer F.Cu) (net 6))
 (segment (start 41.43375 43.02125) (end 43.4975 40.9575) (width 3.175) (layer F.Cu) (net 6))
 (segment (start 43.4975 40.9575) (end 43.4975 36.195) (width 3.175) (layer F.Cu) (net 6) (status 20))
 (segment (start 43.4975 40.9575) (end 43.4975 36.195) (width 3.175) (layer B.Cu) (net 6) (status 20))
 (segment (start 41.43375 43.02125) (end 43.4975 40.9575) (width 3.175) (layer B.Cu) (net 6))
 (segment (start 39.9525 40.005) (end 38.82113 40.005) (width 0.508) (layer B.Cu) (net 12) (status 10))
 (segment (start 38.82113 40.005) (end 38.0475 39.23137) (width 0.508) (layer B.Cu) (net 12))
 (segment (start 38.0475 39.23137) (end 38.0475 36.195) (width 0.508) (layer B.Cu) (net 12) (status 20))
 (segment (start 50.4825 43.18) (end 50.4825 42.545) (width 0.508) (layer B.Cu) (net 16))
 (segment (start 48.5775 36.565) (end 48.9475 36.195) (width 0.508) (layer B.Cu) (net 16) (status 30))
 (segment (start 50.4825 42.545) (end 48.5775 40.64) (width 0.508) (layer B.Cu) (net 16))
 (segment (start 48.5775 40.64) (end 48.5775 36.565) (width 0.508) (layer B.Cu) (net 16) (status 20))
 (segment (start 55.5625 35.8775) (end 49.265 35.8775) (width 3.175) (layer B.Cu) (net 16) (status 30))
 (segment (start 49.265 35.8775) (end 48.9475 36.195) (width 2.54) (layer B.Cu) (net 16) (status 30))
 (segment (start 55.5625 35.8775) (end 49.265 35.8775) (width 3.175) (layer F.Cu) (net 16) (status 30))
 (segment (start 49.265 35.8775) (end 48.9475 36.195) (width 2.54) (layer F.Cu) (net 16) (status 30))
 (segment (start 50.4825 43.18) (end 50.4825 53.4605) (width 0.508) (layer F.Cu) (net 16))
 (segment (start 50.4825 53.4605) (end 51.3145 54.2925) (width 0.508) (layer F.Cu) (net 16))
 (segment (start 51.3145 54.2925) (end 52.705 54.2925) (width 0.508) (layer F.Cu) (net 16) (status 20))
 (via (at 50.4825 43.18) (size 0.6) (drill 0.4) (layers F.Cu B.Cu) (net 16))
 (segment (start 52.6225 54.2925) (end 53.0225 54.2925) (width 0.508) (layer F.Cu) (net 16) (status 30))
 (segment (start 60.325 64.4525) (end 60.325 61.9125) (width 0.508) (layer B.Cu) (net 18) (status 30))
 (segment (start 60.325 51.7525) (end 61.9125 50.165) (width 0.508) (layer B.Cu) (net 5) (status 10))
 (segment (start 61.9125 50.165) (end 61.9125 47.9825) (width 0.508) (layer B.Cu) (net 5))
 (segment (start 61.9125 47.9825) (end 59.9675 46.0375) (width 0.508) (layer B.Cu) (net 5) (status 20))
 (segment (start 59.9675 46.0375) (end 59.9675 44.41) (width 0.508) (layer B.Cu) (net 5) (status 10))
 (segment (start 59.9675 44.41) (end 58.7375 43.18) (width 0.508) (layer B.Cu) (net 5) (status 20))
 (segment (start 58.7375 74.6125) (end 56.8325 76.5175) (width 0.762) (layer B.Cu) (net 11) (status 10))
 (segment (start 56.8325 76.5175) (end 44.1325 76.5175) (width 0.762) (layer B.Cu) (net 11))
 (segment (start 35.8775 69.5325) (end 34.6075 68.2625) (width 0.762) (layer B.Cu) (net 11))
 (segment (start 44.1325 76.5175) (end 37.1475 69.5325) (width 0.762) (layer B.Cu) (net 11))
 (segment (start 37.1475 69.5325) (end 35.8775 69.5325) (width 0.762) (layer B.Cu) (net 11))
 (segment (start 34.6075 68.2625) (end 34.6075 66.3575) (width 0.762) (layer B.Cu) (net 11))
 (segment (start 34.6075 66.3575) (end 36.5125 64.4525) (width 0.762) (layer B.Cu) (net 11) (status 20))
 (segment (start 58.7375 74.6125) (end 62.5475 70.8025) (width 0.762) (layer B.Cu) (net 11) (status 10))
 (segment (start 62.5475 70.8025) (end 65.0875 70.8025) (width 0.762) (layer B.Cu) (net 11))
 (segment (start 65.0875 70.8025) (end 66.04 69.85) (width 0.762) (layer B.Cu) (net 11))
 (segment (start 66.04 69.85) (end 66.04 66.04) (width 0.762) (layer B.Cu) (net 11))
 (segment (start 66.04 66.04) (end 64.4525 64.4525) (width 0.762) (layer B.Cu) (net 11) (status 20))
 (segment (start 52.705 49.2125) (end 51.435 49.2125) (width 0.508) (layer B.Cu) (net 1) (status 10))
 (segment (start 51.435 49.2125) (end 50.8 48.5775) (width 0.508) (layer B.Cu) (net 1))
 (segment (start 50.8 48.5775) (end 50.8 45.085) (width 0.508) (layer B.Cu) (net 1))
 (segment (start 50.8 45.085) (end 50.165 44.45) (width 0.508) (layer B.Cu) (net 1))
 (segment (start 50.165 44.45) (end 48.5775 44.45) (width 0.508) (layer B.Cu) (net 1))
 (segment (start 47.9425 44.45) (end 48.5775 44.45) (width 0.508) (layer B.Cu) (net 1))
 (segment (start 48.5775 44.45) (end 48.5775 43.18) (width 0.508) (layer B.Cu) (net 1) (status 20))
 (segment (start 44.7675 47.625) (end 47.9425 44.45) (width 0.508) (layer B.Cu) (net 1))
 (segment (start 44.7675 47.625) (end 43.18 47.625) (width 0.508) (layer B.Cu) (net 1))
 (segment (start 43.18 47.625) (end 41.5925 46.0375) (width 0.508) (layer B.Cu) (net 1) (status 20))
 (segment (start 52.705 64.4525) (end 54.9275 62.23) (width 0.508) (layer B.Cu) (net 3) (status 10))
 (segment (start 54.9275 62.23) (end 54.9275 58.7375) (width 0.508) (layer B.Cu) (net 3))
 (segment (start 54.9275 58.7375) (end 54.2925 58.1025) (width 0.508) (layer B.Cu) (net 3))
 (segment (start 51.1175 58.1025) (end 49.2125 56.1975) (width 0.508) (layer B.Cu) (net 3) (status 20))
 (segment (start 54.2925 58.1025) (end 51.1175 58.1025) (width 0.508) (layer B.Cu) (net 3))
 (segment (start 39.6875 59.3725) (end 37.798499 57.483499) (width 0.508) (layer B.Cu) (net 17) (status 10))
 (segment (start 37.798499 57.483499) (end 37.798499 51.171499) (width 0.508) (layer B.Cu) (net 17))
 (segment (start 37.798499 51.171499) (end 36.5125 49.8855) (width 0.508) (layer B.Cu) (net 17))
 (segment (start 36.5125 49.8855) (end 36.5125 48.5775) (width 0.508) (layer B.Cu) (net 17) (status 20))
 (segment (start 36.5125 48.5775) (end 39.0525 46.0375) (width 0.508) (layer B.Cu) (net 17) (status 30))
 (segment (start 44.1325 56.1975) (end 45.72 54.61) (width 0.508) (layer B.Cu) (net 2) (status 10))
 (segment (start 45.72 54.61) (end 50.165 54.61) (width 0.508) (layer B.Cu) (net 2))
 (segment (start 50.165 54.61) (end 51.13349 55.57849) (width 0.508) (layer B.Cu) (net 2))
 (segment (start 51.13349 55.57849) (end 53.64151 55.57849) (width 0.508) (layer B.Cu) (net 2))
 (segment (start 53.64151 55.57849) (end 54.2925 54.9275) (width 0.508) (layer B.Cu) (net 2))
 (segment (start 54.2925 54.9275) (end 54.2925 52.6225) (width 0.508) (layer B.Cu) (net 2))
 (segment (start 54.2925 52.6225) (end 53.4225 51.7525) (width 0.508) (layer B.Cu) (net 2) (status 20))
 (segment (start 53.4225 51.7525) (end 52.705 51.7525) (width 0.508) (layer B.Cu) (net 2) (status 30))
 (segment (start 39.0525 56.1975) (end 41.5925 56.1975) (width 0.508) (layer B.Cu) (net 2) (status 30))
 (segment (start 41.5925 56.1975) (end 44.1325 56.1975) (width 0.508) (layer B.Cu) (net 2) (status 30)))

